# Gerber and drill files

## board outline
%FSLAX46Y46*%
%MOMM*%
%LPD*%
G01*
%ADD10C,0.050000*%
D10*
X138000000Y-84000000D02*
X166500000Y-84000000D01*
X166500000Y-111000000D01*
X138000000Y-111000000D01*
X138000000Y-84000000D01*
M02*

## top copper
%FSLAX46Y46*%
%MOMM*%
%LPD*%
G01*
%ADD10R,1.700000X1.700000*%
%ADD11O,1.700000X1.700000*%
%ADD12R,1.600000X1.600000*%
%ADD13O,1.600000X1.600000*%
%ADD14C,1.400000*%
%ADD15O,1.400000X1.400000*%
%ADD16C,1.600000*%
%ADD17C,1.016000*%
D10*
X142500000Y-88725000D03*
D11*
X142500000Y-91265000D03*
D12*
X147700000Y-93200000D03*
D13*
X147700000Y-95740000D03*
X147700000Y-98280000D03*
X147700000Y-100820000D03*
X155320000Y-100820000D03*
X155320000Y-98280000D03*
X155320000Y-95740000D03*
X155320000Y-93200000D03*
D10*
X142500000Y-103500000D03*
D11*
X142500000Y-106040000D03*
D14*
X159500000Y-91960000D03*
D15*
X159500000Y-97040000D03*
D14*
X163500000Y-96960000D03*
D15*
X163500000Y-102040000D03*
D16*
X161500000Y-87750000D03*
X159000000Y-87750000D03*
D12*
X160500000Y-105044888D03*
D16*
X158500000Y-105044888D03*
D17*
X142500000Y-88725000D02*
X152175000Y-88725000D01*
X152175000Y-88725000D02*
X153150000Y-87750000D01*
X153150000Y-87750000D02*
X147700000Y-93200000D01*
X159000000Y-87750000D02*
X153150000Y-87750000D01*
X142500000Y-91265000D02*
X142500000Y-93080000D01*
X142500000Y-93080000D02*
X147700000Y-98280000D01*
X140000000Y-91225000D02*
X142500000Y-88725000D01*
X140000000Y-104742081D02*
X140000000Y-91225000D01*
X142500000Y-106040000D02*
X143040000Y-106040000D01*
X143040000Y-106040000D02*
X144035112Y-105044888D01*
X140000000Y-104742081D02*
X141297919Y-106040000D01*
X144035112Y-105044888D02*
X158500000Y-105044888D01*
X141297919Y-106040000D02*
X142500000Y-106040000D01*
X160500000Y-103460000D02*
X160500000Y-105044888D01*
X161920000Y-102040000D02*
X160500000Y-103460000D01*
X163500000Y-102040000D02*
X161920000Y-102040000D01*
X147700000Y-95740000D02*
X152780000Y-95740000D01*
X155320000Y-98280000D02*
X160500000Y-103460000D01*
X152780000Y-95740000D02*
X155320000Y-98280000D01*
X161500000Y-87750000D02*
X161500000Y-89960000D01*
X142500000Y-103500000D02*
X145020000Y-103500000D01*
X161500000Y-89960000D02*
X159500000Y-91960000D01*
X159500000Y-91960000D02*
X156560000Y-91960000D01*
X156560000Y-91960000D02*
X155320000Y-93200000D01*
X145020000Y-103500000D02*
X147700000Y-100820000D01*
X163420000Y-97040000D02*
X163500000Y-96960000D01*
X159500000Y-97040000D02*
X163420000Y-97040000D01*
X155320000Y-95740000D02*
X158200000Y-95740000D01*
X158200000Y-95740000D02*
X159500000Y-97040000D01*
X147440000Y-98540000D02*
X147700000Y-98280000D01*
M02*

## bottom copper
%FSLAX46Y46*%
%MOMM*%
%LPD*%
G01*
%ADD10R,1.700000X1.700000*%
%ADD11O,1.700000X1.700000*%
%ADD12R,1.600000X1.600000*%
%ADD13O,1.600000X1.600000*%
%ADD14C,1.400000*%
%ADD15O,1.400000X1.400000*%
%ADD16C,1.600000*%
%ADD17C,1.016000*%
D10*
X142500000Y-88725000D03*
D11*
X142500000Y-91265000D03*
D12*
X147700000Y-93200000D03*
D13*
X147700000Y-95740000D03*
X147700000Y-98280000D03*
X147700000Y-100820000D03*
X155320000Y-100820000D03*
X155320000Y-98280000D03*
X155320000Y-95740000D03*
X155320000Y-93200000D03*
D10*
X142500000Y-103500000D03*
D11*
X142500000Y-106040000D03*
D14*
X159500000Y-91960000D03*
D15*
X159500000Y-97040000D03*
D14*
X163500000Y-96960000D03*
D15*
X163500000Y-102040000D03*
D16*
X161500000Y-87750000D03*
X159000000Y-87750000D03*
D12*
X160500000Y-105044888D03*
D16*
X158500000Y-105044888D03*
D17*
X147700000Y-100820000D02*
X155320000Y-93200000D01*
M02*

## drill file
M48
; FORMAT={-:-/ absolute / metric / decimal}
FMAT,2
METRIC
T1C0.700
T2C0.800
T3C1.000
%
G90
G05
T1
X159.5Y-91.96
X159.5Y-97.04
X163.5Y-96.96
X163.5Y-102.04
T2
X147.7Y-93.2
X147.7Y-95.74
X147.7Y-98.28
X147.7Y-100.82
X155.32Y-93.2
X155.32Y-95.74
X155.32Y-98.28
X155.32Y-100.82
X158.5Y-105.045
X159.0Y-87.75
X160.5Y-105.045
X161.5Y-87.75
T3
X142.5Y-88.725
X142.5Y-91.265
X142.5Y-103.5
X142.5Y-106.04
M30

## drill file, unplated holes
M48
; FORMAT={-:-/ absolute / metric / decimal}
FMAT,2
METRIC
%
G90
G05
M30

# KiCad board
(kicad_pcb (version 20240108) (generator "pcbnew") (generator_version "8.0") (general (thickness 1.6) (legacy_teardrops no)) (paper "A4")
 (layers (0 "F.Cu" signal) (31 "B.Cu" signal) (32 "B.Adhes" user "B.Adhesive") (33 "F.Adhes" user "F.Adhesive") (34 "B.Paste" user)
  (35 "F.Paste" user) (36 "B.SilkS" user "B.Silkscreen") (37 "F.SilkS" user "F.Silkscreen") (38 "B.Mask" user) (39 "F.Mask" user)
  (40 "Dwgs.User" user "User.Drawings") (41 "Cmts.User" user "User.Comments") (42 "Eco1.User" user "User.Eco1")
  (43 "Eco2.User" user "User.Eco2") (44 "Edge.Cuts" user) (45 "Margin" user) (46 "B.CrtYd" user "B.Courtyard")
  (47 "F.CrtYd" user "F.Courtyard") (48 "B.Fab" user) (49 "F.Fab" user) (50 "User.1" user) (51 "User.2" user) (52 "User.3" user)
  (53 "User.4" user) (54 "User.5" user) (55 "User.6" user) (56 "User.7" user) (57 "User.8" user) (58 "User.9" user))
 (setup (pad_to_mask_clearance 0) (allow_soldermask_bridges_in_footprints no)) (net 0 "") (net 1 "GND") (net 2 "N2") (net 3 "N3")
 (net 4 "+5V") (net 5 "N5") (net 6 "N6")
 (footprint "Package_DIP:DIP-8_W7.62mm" (layer "F.Cu") (at 147.7 93.2)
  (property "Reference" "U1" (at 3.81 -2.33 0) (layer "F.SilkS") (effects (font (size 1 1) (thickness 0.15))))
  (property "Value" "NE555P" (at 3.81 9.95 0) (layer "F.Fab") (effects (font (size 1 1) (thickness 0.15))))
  (pad "1" thru_hole rect (at 0 0) (size 1.6 1.6) (drill 0.8) (layers "*.Cu" "*.Mask") (remove_unused_layers no) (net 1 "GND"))
  (pad "2" thru_hole oval (at 0 2.54) (size 1.6 1.6) (drill 0.8) (layers "*.Cu" "*.Mask") (remove_unused_layers no) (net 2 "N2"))
  (pad "3" thru_hole oval (at 0 5.08) (size 1.6 1.6) (drill 0.8) (layers "*.Cu" "*.Mask") (remove_unused_layers no) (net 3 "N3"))
  (pad "4" thru_hole oval (at 0 7.62) (size 1.6 1.6) (drill 0.8) (layers "*.Cu" "*.Mask") (remove_unused_layers no) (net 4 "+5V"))
  (pad "5" thru_hole oval (at 7.62 7.62) (size 1.6 1.6) (drill 0.8) (layers "*.Cu" "*.Mask") (remove_unused_layers no) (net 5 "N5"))
  (pad "6" thru_hole oval (at 7.62 5.08) (size 1.6 1.6) (drill 0.8) (layers "*.Cu" "*.Mask") (remove_unused_layers no) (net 2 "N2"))
  (pad "7" thru_hole oval (at 7.62 2.54) (size 1.6 1.6) (drill 0.8) (layers "*.Cu" "*.Mask") (remove_unused_layers no) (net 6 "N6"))
  (pad "8" thru_hole oval (at 7.62 0) (size 1.6 1.6) (drill 0.8) (layers "*.Cu" "*.Mask") (remove_unused_layers no) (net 4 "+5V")))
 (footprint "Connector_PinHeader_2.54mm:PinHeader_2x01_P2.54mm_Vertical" (layer "F.Cu") (at 142.5 103.5 -90)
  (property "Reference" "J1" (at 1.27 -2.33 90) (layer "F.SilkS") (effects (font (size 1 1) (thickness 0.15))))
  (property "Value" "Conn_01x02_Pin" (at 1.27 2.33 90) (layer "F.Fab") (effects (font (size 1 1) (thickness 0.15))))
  (pad "1" thru_hole rect (at 0 0 270) (size 1.7 1.7) (drill 1) (layers "*.Cu" "*.Mask") (remove_unused_layers no) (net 4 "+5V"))
  (pad "2" thru_hole oval (at 2.54 0 270) (size 1.7 1.7) (drill 1) (layers "*.Cu" "*.Mask") (remove_unused_layers no) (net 1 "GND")))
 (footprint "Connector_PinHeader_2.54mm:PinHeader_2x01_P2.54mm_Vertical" (layer "F.Cu") (at 142.5 88.725 -90)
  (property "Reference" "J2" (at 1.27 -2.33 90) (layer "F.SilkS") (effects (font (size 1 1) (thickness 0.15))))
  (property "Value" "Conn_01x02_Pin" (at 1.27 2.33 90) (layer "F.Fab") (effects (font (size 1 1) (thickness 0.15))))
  (pad "1" thru_hole rect (at 0 0 270) (size 1.7 1.7) (drill 1) (layers "*.Cu" "*.Mask") (remove_unused_layers no) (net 1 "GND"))
  (pad "2" thru_hole oval (at 2.54 0 270) (size 1.7 1.7) (drill 1) (layers "*.Cu" "*.Mask") (remove_unused_layers no) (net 3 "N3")))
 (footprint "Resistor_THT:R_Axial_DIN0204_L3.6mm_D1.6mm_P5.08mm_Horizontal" (layer "F.Cu") (at 159.5 91.96 -90)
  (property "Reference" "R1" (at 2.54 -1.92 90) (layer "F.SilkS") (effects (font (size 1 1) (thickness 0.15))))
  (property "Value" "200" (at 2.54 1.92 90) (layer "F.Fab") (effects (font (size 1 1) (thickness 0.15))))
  (pad "1" thru_hole circle (at 0 0 270) (size 1.4 1.4) (drill 0.7) (layers "*.Cu" "*.Mask") (remove_unused_layers no) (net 4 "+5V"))
  (pad "2" thru_hole oval (at 5.08 0 270) (size 1.4 1.4) (drill 0.7) (layers "*.Cu" "*.Mask") (remove_unused_layers no) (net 6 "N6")))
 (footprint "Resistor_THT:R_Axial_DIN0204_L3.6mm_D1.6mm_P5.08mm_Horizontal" (layer "F.Cu") (at 163.5 96.96 -90)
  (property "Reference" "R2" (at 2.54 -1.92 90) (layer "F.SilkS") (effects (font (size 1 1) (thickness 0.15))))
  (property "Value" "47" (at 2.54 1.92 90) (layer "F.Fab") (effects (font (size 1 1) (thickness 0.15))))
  (pad "1" thru_hole circle (at 0 0 270) (size 1.4 1.4) (drill 0.7) (layers "*.Cu" "*.Mask") (remove_unused_layers no) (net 6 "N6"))
  (pad "2" thru_hole oval (at 5.08 0 270) (size 1.4 1.4) (drill 0.7) (layers "*.Cu" "*.Mask") (remove_unused_layers no) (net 2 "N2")))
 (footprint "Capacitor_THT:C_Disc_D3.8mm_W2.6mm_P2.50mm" (layer "F.Cu") (at 161.5 87.75 180)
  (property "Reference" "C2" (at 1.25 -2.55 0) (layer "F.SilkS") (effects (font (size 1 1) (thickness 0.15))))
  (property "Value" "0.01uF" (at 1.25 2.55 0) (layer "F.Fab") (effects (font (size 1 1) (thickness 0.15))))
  (pad "1" thru_hole circle (at 0 0 180) (size 1.6 1.6) (drill 0.8) (layers "*.Cu" "*.Mask") (remove_unused_layers no) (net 4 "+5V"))
  (pad "2" thru_hole circle (at 2.5 0 180) (size 1.6 1.6) (drill 0.8) (layers "*.Cu" "*.Mask") (remove_unused_layers no) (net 1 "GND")))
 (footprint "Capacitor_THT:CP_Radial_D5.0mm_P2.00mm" (layer "F.Cu") (at 160.5 105.044888 180)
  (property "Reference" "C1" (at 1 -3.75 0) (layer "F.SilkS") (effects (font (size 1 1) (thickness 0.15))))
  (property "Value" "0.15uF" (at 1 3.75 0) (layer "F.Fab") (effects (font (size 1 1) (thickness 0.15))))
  (pad "1" thru_hole rect (at 0 0 180) (size 1.6 1.6) (drill 0.8) (layers "*.Cu" "*.Mask") (remove_unused_layers no) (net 2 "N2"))
  (pad "2" thru_hole circle (at 2 0 180) (size 1.6 1.6) (drill 0.8) (layers "*.Cu" "*.Mask") (remove_unused_layers no) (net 1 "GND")))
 (gr_rect (start 138 84) (end 166.5 111) (stroke (width 0.05) (type default)) (fill none) (layer "Edge.Cuts"))
 (segment (start 142.5 106.04) (end 143.04 106.04) (width 1.016) (layer "F.Cu") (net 1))
 (segment (start 142.5 88.725) (end 152.175 88.725) (width 1.016) (layer "F.Cu") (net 1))
 (segment (start 153.15 87.75) (end 147.7 93.2) (width 1.016) (layer "F.Cu") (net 1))
 (segment (start 143.04 106.04) (end 144.035112 105.044888) (width 1.016) (layer "F.Cu") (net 1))
 (segment (start 152.175 88.725) (end 153.15 87.75) (width 1.016) (layer "F.Cu") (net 1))
 (segment (start 140 91.225) (end 142.5 88.725) (width 1.016) (layer "F.Cu") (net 1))
 (segment (start 140 104.742081) (end 141.297919 106.04) (width 1.016) (layer "F.Cu") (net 1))
 (segment (start 144.035112 105.044888) (end 158.5 105.044888) (width 1.016) (layer "F.Cu") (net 1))
 (segment (start 159 87.75) (end 153.15 87.75) (width 1.016) (layer "F.Cu") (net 1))
 (segment (start 140 104.742081) (end 140 91.225) (width 1.016) (layer "F.Cu") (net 1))
 (segment (start 141.297919 106.04) (end 142.5 106.04) (width 1.016) (layer "F.Cu") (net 1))
 (segment (start 160.5 103.46) (end 160.5 105.044888) (width 1.016) (layer "F.Cu") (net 2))
 (segment (start 161.92 102.04) (end 160.5 103.46) (width 1.016) (layer "F.Cu") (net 2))
 (segment (start 163.5 102.04) (end 161.92 102.04) (width 1.016) (layer "F.Cu") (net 2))
 (segment (start 147.7 95.74) (end 152.78 95.74) (width 1.016) (layer "F.Cu") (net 2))
 (segment (start 155.32 98.28) (end 160.5 103.46) (width 1.016) (layer "F.Cu") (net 2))
 (segment (start 152.78 95.74) (end 155.32 98.28) (width 1.016) (layer "F.Cu") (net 2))
 (segment (start 161.5 87.75) (end 161.5 89.96) (width 1.016) (layer "F.Cu") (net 4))
 (segment (start 142.5 103.5) (end 145.02 103.5) (width 1.016) (layer "F.Cu") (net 4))
 (segment (start 161.5 89.96) (end 159.5 91.96) (width 1.016) (layer "F.Cu") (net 4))
 (segment (start 159.5 91.96) (end 156.56 91.96) (width 1.016) (layer "F.Cu") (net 4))
 (segment (start 156.56 91.96) (end 155.32 93.2) (width 1.016) (layer "F.Cu") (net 4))
 (segment (start 145.02 103.5) (end 147.7 100.82) (width 1.016) (layer "F.Cu") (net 4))
 (segment (start 147.7 100.82) (end 155.32 93.2) (width 1.016) (layer "B.Cu") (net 4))
 (segment (start 142.5 91.265) (end 142.5 93.08) (width 1.016) (layer "F.Cu") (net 3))
 (segment (start 147.44 98.54) (end 147.7 98.28) (width 1.016) (layer "F.Cu") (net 3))
 (segment (start 142.5 93.08) (end 147.7 98.28) (width 1.016) (layer "F.Cu") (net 3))
 (segment (start 163.42 97.04) (end 163.5 96.96) (width 1.016) (layer "F.Cu") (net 6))
 (segment (start 159.5 97.04) (end 163.42 97.04) (width 1.016) (layer "F.Cu") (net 6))
 (segment (start 155.32 95.74) (end 158.2 95.74) (width 1.016) (layer "F.Cu") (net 6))
 (segment (start 158.2 95.74) (end 159.5 97.04) (width 1.016) (layer "F.Cu") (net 6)))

